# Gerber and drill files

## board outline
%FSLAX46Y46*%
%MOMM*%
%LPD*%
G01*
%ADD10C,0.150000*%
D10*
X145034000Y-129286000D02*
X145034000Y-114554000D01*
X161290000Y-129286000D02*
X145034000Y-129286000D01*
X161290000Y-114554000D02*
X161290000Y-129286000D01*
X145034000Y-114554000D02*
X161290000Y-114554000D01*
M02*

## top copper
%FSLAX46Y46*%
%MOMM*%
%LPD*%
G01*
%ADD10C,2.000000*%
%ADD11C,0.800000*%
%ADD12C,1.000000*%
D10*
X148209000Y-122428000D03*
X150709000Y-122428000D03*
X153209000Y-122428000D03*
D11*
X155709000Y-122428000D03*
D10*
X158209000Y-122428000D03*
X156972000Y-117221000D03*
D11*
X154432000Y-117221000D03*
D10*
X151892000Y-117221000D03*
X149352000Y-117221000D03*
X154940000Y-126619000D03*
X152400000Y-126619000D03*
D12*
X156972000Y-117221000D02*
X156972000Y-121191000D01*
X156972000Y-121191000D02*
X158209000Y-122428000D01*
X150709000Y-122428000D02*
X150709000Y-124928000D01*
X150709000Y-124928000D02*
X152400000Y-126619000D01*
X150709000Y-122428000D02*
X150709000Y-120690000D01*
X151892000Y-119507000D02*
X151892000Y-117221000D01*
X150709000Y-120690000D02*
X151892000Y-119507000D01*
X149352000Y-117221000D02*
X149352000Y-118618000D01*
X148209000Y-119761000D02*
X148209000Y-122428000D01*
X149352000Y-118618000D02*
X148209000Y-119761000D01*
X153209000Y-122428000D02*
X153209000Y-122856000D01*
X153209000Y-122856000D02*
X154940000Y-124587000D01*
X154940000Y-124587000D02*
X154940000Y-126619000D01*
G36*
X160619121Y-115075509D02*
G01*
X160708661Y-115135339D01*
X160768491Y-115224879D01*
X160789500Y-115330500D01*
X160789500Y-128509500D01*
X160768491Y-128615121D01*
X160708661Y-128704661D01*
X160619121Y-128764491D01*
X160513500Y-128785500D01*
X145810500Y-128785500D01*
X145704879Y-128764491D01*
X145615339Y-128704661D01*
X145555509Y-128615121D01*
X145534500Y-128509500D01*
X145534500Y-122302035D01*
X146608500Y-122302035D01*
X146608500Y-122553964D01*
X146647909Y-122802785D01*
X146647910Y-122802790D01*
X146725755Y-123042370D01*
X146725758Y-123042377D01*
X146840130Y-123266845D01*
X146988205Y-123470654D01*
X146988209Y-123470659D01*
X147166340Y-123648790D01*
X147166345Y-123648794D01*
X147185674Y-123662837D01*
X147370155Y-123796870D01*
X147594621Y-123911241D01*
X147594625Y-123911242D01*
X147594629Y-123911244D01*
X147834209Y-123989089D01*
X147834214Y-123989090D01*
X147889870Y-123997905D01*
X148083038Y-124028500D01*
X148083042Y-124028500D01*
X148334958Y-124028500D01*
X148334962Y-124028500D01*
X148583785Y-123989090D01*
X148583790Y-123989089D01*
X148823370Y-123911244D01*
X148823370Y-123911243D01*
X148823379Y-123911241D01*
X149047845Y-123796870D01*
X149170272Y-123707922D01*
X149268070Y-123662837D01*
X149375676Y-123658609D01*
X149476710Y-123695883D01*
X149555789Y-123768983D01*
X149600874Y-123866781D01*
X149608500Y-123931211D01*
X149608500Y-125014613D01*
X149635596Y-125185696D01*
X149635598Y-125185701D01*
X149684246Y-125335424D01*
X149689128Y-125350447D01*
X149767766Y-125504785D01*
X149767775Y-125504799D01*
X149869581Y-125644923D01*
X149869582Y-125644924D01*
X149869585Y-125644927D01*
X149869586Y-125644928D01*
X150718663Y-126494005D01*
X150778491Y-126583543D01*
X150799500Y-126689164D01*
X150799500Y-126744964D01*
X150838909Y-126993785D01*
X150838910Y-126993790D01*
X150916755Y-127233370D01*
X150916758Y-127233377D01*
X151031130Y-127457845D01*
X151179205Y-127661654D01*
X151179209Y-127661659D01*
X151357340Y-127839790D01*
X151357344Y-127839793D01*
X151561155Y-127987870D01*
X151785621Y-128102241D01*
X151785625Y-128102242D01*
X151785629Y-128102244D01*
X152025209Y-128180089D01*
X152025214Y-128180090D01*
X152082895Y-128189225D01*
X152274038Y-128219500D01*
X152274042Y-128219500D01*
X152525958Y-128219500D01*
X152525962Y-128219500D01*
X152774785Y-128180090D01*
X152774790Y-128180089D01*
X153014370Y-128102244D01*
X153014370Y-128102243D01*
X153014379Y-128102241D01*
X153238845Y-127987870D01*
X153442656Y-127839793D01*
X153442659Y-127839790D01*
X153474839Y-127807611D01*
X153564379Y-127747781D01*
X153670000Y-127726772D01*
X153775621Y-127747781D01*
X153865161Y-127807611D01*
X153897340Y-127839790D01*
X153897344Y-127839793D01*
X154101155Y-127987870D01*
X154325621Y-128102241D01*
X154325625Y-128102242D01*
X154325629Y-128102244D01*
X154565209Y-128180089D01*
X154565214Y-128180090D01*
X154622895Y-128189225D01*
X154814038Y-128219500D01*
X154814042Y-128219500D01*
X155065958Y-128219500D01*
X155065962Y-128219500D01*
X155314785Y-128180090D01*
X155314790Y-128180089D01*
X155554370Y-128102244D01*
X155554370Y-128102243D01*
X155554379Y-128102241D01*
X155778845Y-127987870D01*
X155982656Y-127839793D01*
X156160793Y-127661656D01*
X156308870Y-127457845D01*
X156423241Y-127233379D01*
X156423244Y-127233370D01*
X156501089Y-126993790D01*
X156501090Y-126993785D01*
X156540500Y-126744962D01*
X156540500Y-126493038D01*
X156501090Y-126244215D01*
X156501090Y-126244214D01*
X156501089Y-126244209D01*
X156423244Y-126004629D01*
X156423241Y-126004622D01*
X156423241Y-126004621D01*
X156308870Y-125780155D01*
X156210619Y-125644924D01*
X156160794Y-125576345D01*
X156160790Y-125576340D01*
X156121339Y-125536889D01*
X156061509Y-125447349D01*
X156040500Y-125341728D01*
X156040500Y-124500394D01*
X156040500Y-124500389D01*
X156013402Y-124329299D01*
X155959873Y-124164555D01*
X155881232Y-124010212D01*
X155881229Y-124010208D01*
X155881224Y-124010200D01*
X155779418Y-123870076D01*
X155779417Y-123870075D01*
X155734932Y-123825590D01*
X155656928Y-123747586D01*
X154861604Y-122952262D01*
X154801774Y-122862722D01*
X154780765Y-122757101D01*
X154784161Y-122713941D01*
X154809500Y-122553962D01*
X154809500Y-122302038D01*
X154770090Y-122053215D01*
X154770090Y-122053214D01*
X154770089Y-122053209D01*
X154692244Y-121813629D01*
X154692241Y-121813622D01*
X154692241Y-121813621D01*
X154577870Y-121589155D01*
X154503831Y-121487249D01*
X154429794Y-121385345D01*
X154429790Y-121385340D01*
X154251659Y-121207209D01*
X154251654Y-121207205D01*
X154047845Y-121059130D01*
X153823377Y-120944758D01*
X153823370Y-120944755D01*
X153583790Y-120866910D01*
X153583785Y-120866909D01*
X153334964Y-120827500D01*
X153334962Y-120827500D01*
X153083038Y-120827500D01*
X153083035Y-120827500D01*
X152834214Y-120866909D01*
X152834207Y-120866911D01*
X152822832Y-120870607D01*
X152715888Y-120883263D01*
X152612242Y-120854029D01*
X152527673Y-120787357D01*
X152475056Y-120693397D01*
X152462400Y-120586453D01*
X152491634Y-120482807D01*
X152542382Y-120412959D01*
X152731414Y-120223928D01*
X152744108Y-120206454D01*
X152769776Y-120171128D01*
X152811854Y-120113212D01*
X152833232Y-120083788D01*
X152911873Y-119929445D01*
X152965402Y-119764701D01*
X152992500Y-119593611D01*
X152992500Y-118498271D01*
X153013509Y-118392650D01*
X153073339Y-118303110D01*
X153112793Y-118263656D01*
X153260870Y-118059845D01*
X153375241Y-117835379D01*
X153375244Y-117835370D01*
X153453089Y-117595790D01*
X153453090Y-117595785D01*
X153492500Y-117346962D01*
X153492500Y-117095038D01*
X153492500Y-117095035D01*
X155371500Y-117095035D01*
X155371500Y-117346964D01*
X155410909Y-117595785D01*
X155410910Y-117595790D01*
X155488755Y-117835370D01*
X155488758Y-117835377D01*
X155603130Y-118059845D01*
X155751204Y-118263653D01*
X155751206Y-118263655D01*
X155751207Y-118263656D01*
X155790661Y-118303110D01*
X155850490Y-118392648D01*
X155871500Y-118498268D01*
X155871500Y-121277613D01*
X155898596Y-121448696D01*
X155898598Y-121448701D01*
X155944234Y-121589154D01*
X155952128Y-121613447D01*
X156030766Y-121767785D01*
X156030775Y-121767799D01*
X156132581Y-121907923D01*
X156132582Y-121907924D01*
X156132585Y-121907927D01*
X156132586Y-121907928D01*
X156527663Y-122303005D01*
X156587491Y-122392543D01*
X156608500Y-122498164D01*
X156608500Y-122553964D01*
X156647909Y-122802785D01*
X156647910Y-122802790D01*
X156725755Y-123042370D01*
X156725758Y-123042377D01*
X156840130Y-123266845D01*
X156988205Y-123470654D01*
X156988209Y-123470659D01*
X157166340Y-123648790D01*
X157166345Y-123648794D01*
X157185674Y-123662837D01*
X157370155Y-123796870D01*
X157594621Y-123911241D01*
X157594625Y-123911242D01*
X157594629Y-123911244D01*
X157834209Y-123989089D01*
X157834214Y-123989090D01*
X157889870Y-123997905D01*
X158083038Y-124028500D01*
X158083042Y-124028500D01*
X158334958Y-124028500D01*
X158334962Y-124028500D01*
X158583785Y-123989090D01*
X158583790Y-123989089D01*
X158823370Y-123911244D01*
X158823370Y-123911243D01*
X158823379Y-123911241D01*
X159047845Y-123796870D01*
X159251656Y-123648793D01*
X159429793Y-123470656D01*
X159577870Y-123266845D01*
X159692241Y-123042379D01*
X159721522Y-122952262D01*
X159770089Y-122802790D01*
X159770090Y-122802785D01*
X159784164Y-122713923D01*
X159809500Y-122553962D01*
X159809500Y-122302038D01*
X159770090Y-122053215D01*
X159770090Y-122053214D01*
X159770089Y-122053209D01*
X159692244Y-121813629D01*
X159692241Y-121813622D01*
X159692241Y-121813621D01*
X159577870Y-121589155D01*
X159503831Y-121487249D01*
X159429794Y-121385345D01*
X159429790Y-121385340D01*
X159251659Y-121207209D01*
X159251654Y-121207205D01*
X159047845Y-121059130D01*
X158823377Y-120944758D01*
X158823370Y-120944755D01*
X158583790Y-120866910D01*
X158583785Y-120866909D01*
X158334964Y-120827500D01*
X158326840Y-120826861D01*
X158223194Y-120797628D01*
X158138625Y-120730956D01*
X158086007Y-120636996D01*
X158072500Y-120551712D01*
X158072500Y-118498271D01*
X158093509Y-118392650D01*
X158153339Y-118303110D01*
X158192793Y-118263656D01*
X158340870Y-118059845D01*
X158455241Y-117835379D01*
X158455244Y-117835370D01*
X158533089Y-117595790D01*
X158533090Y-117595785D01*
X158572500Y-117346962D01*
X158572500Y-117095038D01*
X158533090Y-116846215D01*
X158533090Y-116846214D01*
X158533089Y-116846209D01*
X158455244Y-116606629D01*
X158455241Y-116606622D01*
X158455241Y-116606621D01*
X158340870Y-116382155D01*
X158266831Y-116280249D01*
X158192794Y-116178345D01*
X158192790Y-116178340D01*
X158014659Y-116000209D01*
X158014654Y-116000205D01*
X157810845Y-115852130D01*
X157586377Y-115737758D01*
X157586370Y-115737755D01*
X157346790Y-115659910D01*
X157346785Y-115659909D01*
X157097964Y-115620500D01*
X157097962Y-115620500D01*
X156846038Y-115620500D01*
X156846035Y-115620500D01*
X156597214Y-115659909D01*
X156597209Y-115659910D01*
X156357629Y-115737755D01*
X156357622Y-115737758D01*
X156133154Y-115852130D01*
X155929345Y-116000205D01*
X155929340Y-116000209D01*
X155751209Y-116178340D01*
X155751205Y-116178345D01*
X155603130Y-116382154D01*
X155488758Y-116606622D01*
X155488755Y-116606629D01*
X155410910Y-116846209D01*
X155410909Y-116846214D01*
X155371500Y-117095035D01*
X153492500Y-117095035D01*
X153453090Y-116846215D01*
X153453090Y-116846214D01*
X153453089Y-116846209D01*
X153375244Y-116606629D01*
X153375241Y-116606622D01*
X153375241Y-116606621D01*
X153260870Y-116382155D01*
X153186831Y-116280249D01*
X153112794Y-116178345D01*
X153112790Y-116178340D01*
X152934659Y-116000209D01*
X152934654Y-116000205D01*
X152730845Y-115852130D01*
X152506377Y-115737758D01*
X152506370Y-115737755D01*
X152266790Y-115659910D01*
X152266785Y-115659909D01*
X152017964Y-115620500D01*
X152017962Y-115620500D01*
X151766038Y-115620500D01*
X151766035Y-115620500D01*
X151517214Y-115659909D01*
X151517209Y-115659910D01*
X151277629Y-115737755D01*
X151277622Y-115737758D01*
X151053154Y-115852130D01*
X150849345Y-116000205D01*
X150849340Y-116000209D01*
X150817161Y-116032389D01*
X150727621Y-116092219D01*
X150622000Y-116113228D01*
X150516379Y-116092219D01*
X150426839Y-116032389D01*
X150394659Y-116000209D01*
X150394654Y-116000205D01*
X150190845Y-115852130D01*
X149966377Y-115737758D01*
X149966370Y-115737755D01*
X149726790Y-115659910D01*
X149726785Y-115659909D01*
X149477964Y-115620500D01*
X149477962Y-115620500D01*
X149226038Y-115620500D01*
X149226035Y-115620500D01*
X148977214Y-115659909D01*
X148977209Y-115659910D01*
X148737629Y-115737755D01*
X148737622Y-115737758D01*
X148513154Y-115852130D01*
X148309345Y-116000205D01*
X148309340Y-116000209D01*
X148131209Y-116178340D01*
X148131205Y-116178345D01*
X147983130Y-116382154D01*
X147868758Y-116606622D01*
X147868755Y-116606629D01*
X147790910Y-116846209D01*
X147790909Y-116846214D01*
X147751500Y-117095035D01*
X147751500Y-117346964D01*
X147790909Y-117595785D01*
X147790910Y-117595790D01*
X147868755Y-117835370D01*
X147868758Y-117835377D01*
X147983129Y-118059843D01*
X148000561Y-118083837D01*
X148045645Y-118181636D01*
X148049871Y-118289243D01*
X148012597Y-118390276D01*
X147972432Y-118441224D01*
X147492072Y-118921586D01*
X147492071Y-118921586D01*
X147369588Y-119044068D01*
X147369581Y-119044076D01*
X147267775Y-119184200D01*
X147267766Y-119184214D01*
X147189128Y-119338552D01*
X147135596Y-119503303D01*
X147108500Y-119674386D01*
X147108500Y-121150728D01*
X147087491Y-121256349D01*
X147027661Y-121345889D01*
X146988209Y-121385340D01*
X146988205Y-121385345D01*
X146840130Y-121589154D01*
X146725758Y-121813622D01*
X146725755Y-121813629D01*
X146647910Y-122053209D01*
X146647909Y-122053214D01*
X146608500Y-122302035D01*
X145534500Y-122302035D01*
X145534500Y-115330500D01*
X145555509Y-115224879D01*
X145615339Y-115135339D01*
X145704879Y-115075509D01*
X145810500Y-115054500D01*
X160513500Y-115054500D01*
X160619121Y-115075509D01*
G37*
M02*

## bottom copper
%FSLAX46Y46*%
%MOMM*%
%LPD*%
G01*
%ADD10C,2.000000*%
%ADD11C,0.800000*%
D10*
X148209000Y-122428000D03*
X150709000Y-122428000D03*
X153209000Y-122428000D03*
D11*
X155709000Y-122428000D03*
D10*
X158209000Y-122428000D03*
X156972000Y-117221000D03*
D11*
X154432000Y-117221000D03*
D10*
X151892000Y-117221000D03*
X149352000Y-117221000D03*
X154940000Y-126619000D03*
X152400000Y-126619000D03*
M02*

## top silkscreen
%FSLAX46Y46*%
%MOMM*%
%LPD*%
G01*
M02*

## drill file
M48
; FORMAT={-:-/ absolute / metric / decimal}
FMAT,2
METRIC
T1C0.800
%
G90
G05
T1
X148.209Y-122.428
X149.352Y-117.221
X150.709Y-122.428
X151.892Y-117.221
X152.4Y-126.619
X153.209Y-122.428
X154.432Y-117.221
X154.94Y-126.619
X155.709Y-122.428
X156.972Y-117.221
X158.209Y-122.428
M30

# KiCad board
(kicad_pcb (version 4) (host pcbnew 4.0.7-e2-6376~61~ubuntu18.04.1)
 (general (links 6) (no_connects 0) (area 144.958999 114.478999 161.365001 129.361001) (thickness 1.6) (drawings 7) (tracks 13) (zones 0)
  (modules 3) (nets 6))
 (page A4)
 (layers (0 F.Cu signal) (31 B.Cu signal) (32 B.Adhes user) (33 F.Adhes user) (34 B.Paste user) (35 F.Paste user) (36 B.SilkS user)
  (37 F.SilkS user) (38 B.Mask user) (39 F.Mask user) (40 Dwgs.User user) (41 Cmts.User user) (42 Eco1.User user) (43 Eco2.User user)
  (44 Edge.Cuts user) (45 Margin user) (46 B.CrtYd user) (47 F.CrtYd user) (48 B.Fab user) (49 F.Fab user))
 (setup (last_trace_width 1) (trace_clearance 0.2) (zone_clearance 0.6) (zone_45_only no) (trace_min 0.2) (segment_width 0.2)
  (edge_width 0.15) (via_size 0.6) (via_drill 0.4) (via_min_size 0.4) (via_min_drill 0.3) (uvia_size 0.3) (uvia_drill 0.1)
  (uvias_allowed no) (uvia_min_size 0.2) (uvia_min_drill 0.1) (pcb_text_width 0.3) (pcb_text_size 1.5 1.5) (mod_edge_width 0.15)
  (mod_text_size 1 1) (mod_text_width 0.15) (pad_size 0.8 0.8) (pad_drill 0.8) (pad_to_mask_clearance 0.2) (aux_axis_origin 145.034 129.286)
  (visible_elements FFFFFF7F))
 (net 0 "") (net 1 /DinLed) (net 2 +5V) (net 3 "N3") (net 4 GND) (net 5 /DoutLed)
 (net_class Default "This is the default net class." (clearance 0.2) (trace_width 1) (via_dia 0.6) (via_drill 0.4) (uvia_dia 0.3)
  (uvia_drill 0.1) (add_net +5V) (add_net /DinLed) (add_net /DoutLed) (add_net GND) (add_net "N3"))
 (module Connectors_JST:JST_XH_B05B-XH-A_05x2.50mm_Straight (layer B.Cu) (at 148.209 122.428)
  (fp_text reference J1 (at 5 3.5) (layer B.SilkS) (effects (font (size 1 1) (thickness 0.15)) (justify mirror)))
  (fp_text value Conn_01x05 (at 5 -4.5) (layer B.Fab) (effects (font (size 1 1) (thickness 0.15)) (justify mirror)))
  (pad 1 thru_hole circle (at 0 0) (size 2 2) (drill 0.8) (layers *.Cu *.Mask) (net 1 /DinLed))
  (pad 2 thru_hole circle (at 2.5 0) (size 2 2) (drill 0.8) (layers *.Cu *.Mask) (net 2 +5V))
  (pad 3 thru_hole circle (at 5 0) (size 2 2) (drill 0.8) (layers *.Cu *.Mask) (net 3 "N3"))
  (pad 4 thru_hole circle (at 7.5 0) (size 0.8 0.8) (drill 0.8) (layers *.Cu *.Mask) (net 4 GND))
  (pad 5 thru_hole circle (at 10 0) (size 2 2) (drill 0.8) (layers *.Cu *.Mask) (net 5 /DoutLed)))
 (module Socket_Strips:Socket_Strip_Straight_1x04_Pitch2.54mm (layer B.Cu) (at 156.972 117.221 90)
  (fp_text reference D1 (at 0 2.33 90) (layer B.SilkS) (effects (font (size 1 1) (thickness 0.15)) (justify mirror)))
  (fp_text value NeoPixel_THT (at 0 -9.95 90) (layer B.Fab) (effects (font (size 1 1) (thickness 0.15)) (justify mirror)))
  (pad 1 thru_hole circle (at 0 0 90) (size 2 2) (drill 0.8) (layers *.Cu *.Mask) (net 5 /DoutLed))
  (pad 2 thru_hole circle (at 0 -2.54 90) (size 0.8 0.8) (drill 0.8) (layers *.Cu *.Mask) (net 4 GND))
  (pad 3 thru_hole circle (at 0 -5.08 90) (size 2 2) (drill 0.8) (layers *.Cu *.Mask) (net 2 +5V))
  (pad 4 thru_hole circle (at 0 -7.62 90) (size 2 2) (drill 0.8) (layers *.Cu *.Mask) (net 1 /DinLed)))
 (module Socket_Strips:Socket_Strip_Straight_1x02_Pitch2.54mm (layer B.Cu) (at 154.94 126.619 90)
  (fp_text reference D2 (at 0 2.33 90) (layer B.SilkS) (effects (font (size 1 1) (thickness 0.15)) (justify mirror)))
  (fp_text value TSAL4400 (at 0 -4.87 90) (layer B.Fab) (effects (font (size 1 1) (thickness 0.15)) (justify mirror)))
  (pad 1 thru_hole circle (at 0 0 90) (size 2 2) (drill 0.8) (layers *.Cu *.Mask) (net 3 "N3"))
  (pad 2 thru_hole circle (at 0 -2.54 90) (size 2 2) (drill 0.8) (layers *.Cu *.Mask) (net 2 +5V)))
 (gr_line (start 145.034 129.286) (end 145.034 114.554) (angle 90) (layer Edge.Cuts) (width 0.15))
 (gr_line (start 161.29 129.286) (end 145.034 129.286) (angle 90) (layer Edge.Cuts) (width 0.15))
 (gr_line (start 161.29 114.554) (end 161.29 129.286) (angle 90) (layer Edge.Cuts) (width 0.15))
 (gr_line (start 145.034 114.554) (end 161.29 114.554) (angle 90) (layer Edge.Cuts) (width 0.15))
 (segment (start 156.972 117.221) (end 156.972 121.191) (width 1) (layer F.Cu) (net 5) (status 400000))
 (segment (start 156.972 121.191) (end 158.209 122.428) (width 1) (layer F.Cu) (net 5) (status 800000))
 (segment (start 150.709 122.428) (end 150.709 124.928) (width 1) (layer F.Cu) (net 2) (status 400000))
 (segment (start 150.709 124.928) (end 152.4 126.619) (width 1) (layer F.Cu) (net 2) (status 800000))
 (segment (start 150.709 122.428) (end 150.709 120.69) (width 1) (layer F.Cu) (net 2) (status 400000))
 (segment (start 151.892 119.507) (end 151.892 117.221) (width 1) (layer F.Cu) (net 2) (status 800000))
 (segment (start 150.709 120.69) (end 151.892 119.507) (width 1) (layer F.Cu) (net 2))
 (segment (start 149.352 117.221) (end 149.352 118.618) (width 1) (layer F.Cu) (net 1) (status 400000))
 (segment (start 148.209 119.761) (end 148.209 122.428) (width 1) (layer F.Cu) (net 1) (status 800000))
 (segment (start 149.352 118.618) (end 148.209 119.761) (width 1) (layer F.Cu) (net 1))
 (segment (start 153.209 122.428) (end 153.209 122.856) (width 1) (layer F.Cu) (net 3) (status C00000))
 (segment (start 153.209 122.856) (end 154.94 124.587) (width 1) (layer F.Cu) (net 3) (status 400000))
 (segment (start 154.94 124.587) (end 154.94 126.619) (width 1) (layer F.Cu) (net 3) (status 800000))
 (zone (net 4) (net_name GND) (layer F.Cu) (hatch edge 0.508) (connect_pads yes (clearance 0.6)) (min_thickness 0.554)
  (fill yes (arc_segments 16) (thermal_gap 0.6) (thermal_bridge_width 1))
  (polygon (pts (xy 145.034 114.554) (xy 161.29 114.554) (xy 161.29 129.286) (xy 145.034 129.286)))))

